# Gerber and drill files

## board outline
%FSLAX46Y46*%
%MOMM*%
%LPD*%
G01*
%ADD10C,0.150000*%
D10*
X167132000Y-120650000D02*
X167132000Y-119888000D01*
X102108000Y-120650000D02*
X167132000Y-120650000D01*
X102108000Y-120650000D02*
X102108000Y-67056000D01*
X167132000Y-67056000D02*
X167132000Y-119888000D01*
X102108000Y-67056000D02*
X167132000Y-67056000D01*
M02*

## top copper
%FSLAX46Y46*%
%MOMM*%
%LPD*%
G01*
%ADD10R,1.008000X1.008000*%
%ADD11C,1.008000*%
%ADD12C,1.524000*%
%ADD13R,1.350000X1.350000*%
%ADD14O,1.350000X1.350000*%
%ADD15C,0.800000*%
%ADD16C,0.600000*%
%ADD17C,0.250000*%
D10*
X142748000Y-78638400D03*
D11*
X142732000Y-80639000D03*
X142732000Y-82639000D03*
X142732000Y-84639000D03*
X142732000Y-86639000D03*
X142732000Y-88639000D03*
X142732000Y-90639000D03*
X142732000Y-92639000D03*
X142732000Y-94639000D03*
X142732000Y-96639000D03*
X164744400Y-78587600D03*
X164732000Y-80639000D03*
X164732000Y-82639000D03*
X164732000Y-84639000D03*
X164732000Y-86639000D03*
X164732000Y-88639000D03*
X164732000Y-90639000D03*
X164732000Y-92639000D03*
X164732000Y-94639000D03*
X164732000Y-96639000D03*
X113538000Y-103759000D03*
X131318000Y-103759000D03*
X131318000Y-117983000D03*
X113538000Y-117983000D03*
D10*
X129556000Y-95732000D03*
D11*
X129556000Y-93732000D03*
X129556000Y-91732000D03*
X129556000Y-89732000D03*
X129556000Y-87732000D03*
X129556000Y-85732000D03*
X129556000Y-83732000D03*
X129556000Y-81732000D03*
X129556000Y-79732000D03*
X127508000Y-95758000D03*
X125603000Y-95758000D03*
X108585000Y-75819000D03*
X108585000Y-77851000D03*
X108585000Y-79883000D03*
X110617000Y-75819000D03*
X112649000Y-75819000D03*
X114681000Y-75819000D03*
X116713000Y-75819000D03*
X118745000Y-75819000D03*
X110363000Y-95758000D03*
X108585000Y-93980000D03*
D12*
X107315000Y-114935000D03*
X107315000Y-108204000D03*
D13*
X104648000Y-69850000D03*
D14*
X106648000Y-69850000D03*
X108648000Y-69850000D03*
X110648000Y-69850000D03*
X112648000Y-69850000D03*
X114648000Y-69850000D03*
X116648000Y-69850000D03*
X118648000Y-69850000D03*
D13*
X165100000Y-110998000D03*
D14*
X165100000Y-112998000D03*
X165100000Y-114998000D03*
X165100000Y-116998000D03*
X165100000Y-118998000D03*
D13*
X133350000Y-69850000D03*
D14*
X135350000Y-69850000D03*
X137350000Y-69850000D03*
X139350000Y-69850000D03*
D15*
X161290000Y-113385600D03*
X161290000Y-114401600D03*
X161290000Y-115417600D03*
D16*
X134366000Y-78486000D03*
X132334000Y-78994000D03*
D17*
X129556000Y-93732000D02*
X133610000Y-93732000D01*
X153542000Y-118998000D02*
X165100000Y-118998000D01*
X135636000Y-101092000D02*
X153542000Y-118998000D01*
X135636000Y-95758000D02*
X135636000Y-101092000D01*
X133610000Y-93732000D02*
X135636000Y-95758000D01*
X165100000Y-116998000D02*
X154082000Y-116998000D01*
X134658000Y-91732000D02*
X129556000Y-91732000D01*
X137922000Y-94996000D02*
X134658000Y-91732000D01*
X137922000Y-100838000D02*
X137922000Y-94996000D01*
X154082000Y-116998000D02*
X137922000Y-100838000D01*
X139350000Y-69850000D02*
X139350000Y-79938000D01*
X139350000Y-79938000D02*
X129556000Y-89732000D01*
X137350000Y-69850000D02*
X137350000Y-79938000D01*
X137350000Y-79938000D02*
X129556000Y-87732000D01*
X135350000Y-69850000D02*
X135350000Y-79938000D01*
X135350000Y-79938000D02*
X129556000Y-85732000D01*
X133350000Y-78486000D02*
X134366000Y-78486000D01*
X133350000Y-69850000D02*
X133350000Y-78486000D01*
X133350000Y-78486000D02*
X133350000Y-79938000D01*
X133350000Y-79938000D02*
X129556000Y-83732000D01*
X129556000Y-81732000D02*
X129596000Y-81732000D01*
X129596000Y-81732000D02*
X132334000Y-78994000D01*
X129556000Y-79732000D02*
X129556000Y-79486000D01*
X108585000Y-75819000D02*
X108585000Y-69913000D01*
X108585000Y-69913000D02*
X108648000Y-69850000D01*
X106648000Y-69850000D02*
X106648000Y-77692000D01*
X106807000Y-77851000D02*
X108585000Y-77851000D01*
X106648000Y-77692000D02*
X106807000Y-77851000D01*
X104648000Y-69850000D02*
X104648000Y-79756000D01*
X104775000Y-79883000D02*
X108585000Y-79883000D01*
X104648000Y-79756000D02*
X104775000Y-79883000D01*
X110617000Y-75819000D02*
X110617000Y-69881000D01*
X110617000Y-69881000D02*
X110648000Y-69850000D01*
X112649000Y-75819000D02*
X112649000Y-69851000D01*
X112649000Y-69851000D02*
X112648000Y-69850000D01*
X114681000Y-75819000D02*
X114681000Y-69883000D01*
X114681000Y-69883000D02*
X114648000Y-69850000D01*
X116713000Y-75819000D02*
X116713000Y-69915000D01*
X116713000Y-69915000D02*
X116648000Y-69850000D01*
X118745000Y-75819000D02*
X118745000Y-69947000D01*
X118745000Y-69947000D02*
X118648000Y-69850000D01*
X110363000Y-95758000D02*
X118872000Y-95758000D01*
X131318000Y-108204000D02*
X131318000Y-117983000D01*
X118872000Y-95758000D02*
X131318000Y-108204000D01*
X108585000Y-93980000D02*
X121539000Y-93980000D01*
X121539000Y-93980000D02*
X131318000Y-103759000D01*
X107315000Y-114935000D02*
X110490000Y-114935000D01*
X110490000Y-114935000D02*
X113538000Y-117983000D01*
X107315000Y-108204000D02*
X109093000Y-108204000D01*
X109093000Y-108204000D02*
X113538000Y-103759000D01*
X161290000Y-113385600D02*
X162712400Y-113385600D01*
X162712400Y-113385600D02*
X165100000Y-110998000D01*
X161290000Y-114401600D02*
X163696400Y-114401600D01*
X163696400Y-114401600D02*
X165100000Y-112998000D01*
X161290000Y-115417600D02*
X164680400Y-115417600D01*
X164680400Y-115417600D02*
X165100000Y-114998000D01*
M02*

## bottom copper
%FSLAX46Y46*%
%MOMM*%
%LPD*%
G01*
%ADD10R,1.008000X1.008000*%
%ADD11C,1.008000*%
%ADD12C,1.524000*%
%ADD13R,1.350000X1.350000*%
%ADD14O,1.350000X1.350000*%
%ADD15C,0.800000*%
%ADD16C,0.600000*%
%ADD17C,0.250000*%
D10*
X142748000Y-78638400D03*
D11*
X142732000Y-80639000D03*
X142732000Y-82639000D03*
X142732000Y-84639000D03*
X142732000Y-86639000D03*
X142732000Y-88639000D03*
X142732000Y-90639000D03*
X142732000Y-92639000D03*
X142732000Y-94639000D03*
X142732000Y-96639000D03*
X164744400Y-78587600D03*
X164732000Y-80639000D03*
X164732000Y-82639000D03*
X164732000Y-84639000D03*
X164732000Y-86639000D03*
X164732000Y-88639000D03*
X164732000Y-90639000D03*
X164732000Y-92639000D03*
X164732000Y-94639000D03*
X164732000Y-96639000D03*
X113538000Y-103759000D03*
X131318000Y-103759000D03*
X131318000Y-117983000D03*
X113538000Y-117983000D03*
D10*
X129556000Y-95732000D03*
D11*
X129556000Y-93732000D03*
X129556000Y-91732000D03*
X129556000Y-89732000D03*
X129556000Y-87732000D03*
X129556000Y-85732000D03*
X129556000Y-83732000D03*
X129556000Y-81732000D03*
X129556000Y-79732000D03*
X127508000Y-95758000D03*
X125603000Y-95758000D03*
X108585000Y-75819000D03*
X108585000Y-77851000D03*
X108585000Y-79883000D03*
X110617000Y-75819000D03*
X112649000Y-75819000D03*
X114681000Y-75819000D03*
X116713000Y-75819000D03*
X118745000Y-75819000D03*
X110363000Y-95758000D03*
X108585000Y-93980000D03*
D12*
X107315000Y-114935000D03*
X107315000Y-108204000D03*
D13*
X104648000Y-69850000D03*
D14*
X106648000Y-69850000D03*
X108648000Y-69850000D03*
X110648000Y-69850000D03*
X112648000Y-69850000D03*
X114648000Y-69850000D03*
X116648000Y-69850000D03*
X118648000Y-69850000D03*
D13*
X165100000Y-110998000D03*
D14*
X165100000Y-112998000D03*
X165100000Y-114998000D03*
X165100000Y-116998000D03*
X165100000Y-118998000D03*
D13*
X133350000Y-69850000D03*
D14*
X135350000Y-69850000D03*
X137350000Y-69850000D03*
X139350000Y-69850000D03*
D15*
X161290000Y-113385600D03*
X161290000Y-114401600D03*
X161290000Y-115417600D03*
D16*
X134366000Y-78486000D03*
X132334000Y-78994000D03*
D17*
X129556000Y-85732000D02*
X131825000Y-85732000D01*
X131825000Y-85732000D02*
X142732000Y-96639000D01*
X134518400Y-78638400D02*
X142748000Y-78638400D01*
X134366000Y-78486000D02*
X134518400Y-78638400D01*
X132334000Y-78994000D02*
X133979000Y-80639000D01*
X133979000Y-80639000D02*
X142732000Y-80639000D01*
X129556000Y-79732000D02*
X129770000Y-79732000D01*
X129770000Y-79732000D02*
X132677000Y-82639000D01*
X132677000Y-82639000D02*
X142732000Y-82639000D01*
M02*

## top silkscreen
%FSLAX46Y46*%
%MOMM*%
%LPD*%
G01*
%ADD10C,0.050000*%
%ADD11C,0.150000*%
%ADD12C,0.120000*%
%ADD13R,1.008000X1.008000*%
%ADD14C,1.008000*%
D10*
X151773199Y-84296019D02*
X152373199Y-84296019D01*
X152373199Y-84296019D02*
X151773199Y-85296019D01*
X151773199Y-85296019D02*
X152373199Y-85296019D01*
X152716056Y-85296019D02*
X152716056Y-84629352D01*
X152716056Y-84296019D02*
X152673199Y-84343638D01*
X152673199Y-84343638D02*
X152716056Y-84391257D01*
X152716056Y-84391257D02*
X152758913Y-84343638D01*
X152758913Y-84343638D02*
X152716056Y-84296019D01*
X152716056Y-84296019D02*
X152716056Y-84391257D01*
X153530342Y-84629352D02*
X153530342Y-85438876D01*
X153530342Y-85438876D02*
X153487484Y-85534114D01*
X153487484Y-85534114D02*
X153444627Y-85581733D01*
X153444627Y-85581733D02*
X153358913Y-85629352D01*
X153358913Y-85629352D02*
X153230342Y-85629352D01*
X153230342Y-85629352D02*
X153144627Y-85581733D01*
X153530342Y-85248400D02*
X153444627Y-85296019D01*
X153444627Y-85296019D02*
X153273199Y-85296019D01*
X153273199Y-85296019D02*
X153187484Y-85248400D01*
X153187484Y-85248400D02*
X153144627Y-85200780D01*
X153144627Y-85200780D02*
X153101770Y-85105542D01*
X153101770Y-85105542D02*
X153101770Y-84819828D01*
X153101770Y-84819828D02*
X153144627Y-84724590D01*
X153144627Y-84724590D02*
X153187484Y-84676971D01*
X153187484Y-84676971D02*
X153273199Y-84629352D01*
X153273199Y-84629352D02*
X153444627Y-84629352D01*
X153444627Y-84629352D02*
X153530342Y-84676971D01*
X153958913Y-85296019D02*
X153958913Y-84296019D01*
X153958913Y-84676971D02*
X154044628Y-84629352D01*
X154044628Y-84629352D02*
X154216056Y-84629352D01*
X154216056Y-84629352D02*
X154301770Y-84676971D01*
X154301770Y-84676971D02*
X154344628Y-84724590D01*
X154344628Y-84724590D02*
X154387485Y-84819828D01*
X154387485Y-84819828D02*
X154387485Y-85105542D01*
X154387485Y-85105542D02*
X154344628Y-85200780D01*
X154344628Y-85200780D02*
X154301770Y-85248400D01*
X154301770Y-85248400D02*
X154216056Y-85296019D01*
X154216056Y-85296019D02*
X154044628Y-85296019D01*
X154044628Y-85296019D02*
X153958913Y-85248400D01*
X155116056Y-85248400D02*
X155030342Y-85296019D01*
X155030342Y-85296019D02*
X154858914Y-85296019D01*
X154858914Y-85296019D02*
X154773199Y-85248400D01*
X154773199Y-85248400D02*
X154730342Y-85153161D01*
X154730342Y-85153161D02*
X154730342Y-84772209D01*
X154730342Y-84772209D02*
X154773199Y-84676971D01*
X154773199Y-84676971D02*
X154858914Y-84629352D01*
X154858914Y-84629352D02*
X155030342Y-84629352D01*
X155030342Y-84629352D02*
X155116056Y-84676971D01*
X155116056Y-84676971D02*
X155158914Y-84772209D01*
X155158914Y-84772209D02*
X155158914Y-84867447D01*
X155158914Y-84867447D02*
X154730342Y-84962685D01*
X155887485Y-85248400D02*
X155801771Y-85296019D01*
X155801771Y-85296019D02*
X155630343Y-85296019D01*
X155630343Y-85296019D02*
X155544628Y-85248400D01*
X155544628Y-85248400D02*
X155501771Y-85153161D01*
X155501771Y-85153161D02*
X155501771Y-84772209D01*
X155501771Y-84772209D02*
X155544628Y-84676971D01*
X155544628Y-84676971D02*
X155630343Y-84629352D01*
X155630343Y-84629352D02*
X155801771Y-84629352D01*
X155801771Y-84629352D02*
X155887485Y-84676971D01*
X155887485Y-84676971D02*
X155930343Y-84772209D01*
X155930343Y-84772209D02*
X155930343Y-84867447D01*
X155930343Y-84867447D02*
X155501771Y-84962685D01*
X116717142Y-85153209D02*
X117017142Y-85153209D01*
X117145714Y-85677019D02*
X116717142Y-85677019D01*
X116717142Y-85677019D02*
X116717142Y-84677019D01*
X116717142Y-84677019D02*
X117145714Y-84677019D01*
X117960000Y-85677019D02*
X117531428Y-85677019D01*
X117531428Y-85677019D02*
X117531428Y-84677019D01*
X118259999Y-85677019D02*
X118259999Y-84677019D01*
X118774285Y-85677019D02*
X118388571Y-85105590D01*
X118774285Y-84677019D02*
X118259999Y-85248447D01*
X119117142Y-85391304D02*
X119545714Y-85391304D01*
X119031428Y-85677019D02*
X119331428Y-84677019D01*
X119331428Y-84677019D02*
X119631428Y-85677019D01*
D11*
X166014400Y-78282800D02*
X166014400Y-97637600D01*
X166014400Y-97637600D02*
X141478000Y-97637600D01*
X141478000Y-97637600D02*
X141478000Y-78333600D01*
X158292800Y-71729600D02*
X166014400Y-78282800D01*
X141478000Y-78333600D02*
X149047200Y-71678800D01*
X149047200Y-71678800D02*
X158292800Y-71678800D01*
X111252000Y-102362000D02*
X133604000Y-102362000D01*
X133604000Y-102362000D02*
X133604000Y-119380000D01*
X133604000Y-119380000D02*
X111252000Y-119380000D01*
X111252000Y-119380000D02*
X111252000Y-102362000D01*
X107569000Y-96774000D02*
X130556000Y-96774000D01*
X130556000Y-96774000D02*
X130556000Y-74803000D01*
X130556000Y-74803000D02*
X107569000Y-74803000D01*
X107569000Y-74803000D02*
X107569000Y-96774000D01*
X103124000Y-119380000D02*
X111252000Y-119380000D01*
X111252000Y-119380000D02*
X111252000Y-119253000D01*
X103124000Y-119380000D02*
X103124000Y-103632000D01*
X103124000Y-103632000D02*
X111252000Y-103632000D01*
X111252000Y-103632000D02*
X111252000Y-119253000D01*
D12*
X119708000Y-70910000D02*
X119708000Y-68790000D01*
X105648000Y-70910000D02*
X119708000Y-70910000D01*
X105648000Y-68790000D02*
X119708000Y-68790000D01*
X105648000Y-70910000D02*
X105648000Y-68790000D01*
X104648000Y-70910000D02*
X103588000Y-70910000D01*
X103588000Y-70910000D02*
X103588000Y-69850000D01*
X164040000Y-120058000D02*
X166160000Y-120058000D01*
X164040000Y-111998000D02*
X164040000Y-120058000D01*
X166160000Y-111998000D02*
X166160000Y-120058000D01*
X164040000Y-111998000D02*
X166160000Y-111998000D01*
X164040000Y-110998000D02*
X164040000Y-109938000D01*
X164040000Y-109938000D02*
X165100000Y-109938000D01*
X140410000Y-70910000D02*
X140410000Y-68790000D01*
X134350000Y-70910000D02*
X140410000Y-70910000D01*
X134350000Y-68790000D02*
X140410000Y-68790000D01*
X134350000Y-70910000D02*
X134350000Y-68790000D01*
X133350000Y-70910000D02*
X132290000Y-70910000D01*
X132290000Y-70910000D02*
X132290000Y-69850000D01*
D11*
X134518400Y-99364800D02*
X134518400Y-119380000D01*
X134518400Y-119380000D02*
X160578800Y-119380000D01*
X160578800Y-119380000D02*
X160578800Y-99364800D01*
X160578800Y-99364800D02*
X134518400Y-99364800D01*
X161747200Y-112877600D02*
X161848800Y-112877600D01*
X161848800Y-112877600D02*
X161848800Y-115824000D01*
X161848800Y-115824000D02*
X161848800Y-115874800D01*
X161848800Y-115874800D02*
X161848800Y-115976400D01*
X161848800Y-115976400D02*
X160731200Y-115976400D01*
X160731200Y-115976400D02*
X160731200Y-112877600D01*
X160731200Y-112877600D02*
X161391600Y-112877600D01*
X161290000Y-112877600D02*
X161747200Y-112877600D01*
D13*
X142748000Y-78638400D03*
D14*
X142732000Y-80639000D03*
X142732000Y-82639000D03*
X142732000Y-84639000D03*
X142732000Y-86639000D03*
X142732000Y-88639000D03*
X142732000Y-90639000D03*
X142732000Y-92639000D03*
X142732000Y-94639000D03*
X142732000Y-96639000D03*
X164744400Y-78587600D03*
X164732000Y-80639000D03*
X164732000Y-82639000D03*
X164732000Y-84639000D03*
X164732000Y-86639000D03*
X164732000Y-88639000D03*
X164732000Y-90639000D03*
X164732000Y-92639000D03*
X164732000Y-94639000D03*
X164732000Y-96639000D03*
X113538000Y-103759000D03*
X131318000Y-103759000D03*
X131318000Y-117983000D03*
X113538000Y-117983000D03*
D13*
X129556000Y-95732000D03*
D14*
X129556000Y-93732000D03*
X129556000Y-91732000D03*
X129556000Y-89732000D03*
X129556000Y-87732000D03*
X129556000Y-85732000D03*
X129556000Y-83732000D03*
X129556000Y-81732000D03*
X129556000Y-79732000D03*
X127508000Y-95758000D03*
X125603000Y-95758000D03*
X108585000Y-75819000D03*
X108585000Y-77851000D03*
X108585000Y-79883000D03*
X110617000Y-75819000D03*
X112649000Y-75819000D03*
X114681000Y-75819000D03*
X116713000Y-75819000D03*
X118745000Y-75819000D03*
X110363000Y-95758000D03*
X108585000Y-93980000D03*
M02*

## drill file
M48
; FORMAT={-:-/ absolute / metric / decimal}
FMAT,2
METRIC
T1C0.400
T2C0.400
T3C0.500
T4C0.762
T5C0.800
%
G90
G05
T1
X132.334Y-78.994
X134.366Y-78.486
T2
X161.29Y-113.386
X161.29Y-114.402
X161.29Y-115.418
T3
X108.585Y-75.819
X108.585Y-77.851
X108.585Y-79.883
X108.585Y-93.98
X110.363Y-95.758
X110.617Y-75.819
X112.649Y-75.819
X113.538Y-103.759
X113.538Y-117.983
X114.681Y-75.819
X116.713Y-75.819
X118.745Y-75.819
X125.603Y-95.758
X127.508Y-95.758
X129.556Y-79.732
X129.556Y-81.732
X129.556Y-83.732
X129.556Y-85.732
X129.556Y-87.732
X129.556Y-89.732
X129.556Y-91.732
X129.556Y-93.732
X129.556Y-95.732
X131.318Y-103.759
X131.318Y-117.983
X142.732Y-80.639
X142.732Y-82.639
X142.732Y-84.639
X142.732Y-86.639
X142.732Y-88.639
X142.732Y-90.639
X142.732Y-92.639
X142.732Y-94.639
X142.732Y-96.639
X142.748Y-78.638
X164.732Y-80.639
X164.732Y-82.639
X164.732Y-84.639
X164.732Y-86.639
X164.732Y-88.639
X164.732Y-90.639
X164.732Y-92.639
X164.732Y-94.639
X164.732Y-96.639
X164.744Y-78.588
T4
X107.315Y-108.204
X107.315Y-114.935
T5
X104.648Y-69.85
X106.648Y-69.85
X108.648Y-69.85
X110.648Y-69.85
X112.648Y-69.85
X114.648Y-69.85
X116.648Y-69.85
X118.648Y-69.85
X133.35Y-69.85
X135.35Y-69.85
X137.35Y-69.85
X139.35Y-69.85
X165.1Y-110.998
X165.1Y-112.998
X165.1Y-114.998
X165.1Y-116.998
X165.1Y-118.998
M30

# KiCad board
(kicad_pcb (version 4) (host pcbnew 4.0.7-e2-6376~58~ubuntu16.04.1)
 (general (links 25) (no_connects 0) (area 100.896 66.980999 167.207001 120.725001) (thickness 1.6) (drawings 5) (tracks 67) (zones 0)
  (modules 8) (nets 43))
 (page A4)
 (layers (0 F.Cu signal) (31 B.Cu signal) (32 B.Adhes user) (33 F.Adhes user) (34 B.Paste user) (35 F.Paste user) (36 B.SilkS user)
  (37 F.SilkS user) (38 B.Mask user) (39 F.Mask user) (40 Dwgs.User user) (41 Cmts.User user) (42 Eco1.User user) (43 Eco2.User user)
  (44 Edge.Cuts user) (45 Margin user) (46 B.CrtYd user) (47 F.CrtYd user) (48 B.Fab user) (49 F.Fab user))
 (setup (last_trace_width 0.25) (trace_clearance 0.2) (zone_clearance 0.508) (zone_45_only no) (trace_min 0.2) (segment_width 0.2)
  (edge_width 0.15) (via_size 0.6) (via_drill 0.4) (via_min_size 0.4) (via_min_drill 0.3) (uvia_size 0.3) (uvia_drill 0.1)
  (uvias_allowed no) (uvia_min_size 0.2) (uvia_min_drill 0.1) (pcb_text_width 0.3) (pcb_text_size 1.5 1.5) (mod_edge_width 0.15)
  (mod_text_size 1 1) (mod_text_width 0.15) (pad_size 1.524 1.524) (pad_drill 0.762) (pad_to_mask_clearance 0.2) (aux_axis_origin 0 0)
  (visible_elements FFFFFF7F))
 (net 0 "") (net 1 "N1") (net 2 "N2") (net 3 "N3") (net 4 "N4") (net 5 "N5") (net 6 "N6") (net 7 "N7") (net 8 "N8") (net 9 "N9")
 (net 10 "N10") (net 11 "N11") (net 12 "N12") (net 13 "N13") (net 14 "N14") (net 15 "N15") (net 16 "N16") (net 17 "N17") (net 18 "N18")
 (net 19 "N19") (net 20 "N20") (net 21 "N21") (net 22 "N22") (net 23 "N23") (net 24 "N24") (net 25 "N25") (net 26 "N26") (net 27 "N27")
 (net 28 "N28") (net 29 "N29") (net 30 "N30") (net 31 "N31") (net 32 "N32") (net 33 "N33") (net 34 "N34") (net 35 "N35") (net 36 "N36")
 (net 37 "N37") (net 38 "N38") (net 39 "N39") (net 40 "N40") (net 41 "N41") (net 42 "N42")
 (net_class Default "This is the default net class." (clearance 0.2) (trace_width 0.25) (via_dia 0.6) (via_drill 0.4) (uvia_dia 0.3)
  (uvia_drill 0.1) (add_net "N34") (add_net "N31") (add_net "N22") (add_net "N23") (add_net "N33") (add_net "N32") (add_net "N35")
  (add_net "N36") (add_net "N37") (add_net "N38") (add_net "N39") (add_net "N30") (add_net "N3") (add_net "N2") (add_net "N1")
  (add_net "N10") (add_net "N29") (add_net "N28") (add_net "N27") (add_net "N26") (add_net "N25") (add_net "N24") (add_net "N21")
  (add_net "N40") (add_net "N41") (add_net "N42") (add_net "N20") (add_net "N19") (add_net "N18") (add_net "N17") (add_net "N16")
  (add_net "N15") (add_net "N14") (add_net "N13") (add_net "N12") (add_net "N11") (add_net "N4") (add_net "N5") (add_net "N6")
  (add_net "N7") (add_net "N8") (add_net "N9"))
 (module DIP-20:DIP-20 (layer F.Cu) (at 141.478 104.648)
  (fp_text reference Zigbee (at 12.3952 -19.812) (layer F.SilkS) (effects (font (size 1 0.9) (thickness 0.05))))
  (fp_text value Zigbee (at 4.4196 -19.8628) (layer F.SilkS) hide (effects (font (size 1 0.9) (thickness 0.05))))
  (fp_line (start 24.5364 -26.3652) (end 24.5364 -7.0104) (layer F.SilkS) (width 0.15))
  (fp_line (start 24.5364 -7.0104) (end 0 -7.0104) (layer F.SilkS) (width 0.15))
  (fp_line (start 0 -7.0104) (end 0 -26.3144) (layer F.SilkS) (width 0.15))
  (fp_line (start 16.8148 -32.9184) (end 24.5364 -26.3652) (layer F.SilkS) (width 0.15))
  (fp_line (start 0 -26.3144) (end 7.5692 -32.9692) (layer F.SilkS) (width 0.15))
  (fp_line (start 7.5692 -32.9692) (end 16.8148 -32.9692) (layer F.SilkS) (width 0.15))
  (pad 1 thru_hole rect (at 1.27 -26.0096) (size 1.008 1.008) (drill 0.5) (layers *.Cu *.Mask F.SilkS) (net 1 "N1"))
  (pad 2 thru_hole circle (at 1.254 -24.009) (size 1.008 1.008) (drill 0.5) (layers *.Cu *.Mask F.SilkS) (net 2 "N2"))
  (pad 3 thru_hole circle (at 1.254 -22.009) (size 1.008 1.008) (drill 0.5) (layers *.Cu *.Mask F.SilkS) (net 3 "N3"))
  (pad 4 thru_hole circle (at 1.254 -20.009) (size 1.008 1.008) (drill 0.5) (layers *.Cu *.Mask F.SilkS) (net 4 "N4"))
  (pad 5 thru_hole circle (at 1.254 -18.009) (size 1.008 1.008) (drill 0.5) (layers *.Cu *.Mask F.SilkS) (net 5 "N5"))
  (pad 6 thru_hole circle (at 1.254 -16.009) (size 1.008 1.008) (drill 0.5) (layers *.Cu *.Mask F.SilkS) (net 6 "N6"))
  (pad 7 thru_hole circle (at 1.254 -14.009) (size 1.008 1.008) (drill 0.5) (layers *.Cu *.Mask F.SilkS) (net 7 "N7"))
  (pad 8 thru_hole circle (at 1.254 -12.009) (size 1.008 1.008) (drill 0.5) (layers *.Cu *.Mask F.SilkS) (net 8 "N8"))
  (pad 9 thru_hole circle (at 1.254 -10.009) (size 1.008 1.008) (drill 0.5) (layers *.Cu *.Mask F.SilkS) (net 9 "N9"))
  (pad 10 thru_hole circle (at 1.254 -8.009) (size 1.008 1.008) (drill 0.5) (layers *.Cu *.Mask F.SilkS) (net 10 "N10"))
  (pad 20 thru_hole circle (at 23.2664 -26.0604) (size 1.008 1.008) (drill 0.5) (layers *.Cu *.Mask F.SilkS) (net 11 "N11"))
  (pad 19 thru_hole circle (at 23.254 -24.009) (size 1.008 1.008) (drill 0.5) (layers *.Cu *.Mask F.SilkS) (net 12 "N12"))
  (pad 18 thru_hole circle (at 23.254 -22.009) (size 1.008 1.008) (drill 0.5) (layers *.Cu *.Mask F.SilkS) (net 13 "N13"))
  (pad 17 thru_hole circle (at 23.254 -20.009) (size 1.008 1.008) (drill 0.5) (layers *.Cu *.Mask F.SilkS) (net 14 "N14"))
  (pad 16 thru_hole circle (at 23.254 -18.009) (size 1.008 1.008) (drill 0.5) (layers *.Cu *.Mask F.SilkS) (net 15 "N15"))
  (pad 15 thru_hole circle (at 23.254 -16.009) (size 1.008 1.008) (drill 0.5) (layers *.Cu *.Mask F.SilkS) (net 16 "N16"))
  (pad 14 thru_hole circle (at 23.254 -14.009) (size 1.008 1.008) (drill 0.5) (layers *.Cu *.Mask F.SilkS) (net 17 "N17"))
  (pad 13 thru_hole circle (at 23.254 -12.009) (size 1.008 1.008) (drill 0.5) (layers *.Cu *.Mask F.SilkS) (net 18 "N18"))
  (pad 12 thru_hole circle (at 23.254 -10.009) (size 1.008 1.008) (drill 0.5) (layers *.Cu *.Mask F.SilkS) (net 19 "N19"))
  (pad 11 thru_hole circle (at 23.254 -8.009) (size 1.008 1.008) (drill 0.5) (layers *.Cu *.Mask F.SilkS) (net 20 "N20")))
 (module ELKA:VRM (layer F.Cu) (at 118.872 100.838)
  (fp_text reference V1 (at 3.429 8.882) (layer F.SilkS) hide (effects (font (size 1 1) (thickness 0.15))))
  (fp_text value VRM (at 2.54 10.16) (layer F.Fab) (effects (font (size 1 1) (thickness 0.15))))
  (fp_line (start -7.62 1.524) (end 14.732 1.524) (layer F.SilkS) (width 0.15))
  (fp_line (start 14.732 1.524) (end 14.732 18.542) (layer F.SilkS) (width 0.15))
  (fp_line (start 14.732 18.542) (end -7.62 18.542) (layer F.SilkS) (width 0.15))
  (fp_line (start -7.62 18.542) (end -7.62 1.524) (layer F.SilkS) (width 0.15))
  (pad 2 thru_hole circle (at -5.334 2.921) (size 1.008 1.008) (drill 0.5) (layers *.Cu *.Mask F.SilkS) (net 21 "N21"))
  (pad 4 thru_hole circle (at 12.446 2.921) (size 1.008 1.008) (drill 0.5) (layers *.Cu *.Mask F.SilkS) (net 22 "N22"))
  (pad 3 thru_hole circle (at 12.446 17.145) (size 1.008 1.008) (drill 0.5) (layers *.Cu *.Mask F.SilkS) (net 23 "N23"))
  (pad 1 thru_hole circle (at -5.334 17.145) (size 1.008 1.008) (drill 0.5) (layers *.Cu *.Mask F.SilkS) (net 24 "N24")))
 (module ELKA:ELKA (layer F.Cu) (at 118.11 72.39 180)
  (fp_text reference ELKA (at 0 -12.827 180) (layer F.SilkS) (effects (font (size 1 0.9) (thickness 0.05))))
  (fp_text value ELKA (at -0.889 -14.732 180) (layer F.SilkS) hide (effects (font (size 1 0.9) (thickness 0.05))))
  (fp_line (start 10.541 -24.384) (end -12.446 -24.384) (layer F.SilkS) (width 0.15))
  (fp_line (start -12.446 -24.384) (end -12.446 -2.413) (layer F.SilkS) (width 0.15))
  (fp_line (start -12.446 -2.413) (end 10.541 -2.413) (layer F.SilkS) (width 0.15))
  (fp_line (start 10.541 -2.413) (end 10.541 -24.384) (layer F.SilkS) (width 0.15))
  (pad I thru_hole rect (at -11.446 -23.342 180) (size 1.008 1.008) (drill 0.5) (layers *.Cu *.Mask F.SilkS) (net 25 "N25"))
  (pad H thru_hole circle (at -11.446 -21.342 180) (size 1.008 1.008) (drill 0.5) (layers *.Cu *.Mask F.SilkS) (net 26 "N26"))
  (pad G thru_hole circle (at -11.446 -19.342 180) (size 1.008 1.008) (drill 0.5) (layers *.Cu *.Mask F.SilkS) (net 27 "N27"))
  (pad F thru_hole circle (at -11.446 -17.342 180) (size 1.008 1.008) (drill 0.5) (layers *.Cu *.Mask F.SilkS) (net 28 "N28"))
  (pad E thru_hole circle (at -11.446 -15.342 180) (size 1.008 1.008) (drill 0.5) (layers *.Cu *.Mask F.SilkS) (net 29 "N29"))
  (pad D thru_hole circle (at -11.446 -13.342 180) (size 1.008 1.008) (drill 0.5) (layers *.Cu *.Mask F.SilkS) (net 10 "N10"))
  (pad C thru_hole circle (at -11.446 -11.342 180) (size 1.008 1.008) (drill 0.5) (layers *.Cu *.Mask F.SilkS) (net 1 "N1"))
  (pad B thru_hole circle (at -11.446 -9.342 180) (size 1.008 1.008) (drill 0.5) (layers *.Cu *.Mask F.SilkS) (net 2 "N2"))
  (pad A thru_hole circle (at -11.446 -7.342 180) (size 1.008 1.008) (drill 0.5) (layers *.Cu *.Mask F.SilkS) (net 3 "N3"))
  (pad 9 thru_hole circle (at -9.398 -23.368 180) (size 1.008 1.008) (drill 0.5) (layers *.Cu *.Mask F.SilkS) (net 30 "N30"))
  (pad 10 thru_hole circle (at -7.493 -23.368 180) (size 1.008 1.008) (drill 0.5) (layers *.Cu *.Mask F.SilkS) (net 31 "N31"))
  (pad 3 thru_hole circle (at 9.525 -3.429 180) (size 1.008 1.008) (drill 0.5) (layers *.Cu *.Mask F.SilkS) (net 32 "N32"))
  (pad 2 thru_hole circle (at 9.525 -5.461 180) (size 1.008 1.008) (drill 0.5) (layers *.Cu *.Mask F.SilkS) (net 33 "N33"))
  (pad 1 thru_hole circle (at 9.525 -7.493 180) (size 1.008 1.008) (drill 0.5) (layers *.Cu *.Mask F.SilkS) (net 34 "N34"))
  (pad 4 thru_hole circle (at 7.493 -3.429 180) (size 1.008 1.008) (drill 0.5) (layers *.Cu *.Mask F.SilkS) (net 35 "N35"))
  (pad 5 thru_hole circle (at 5.461 -3.429 180) (size 1.008 1.008) (drill 0.5) (layers *.Cu *.Mask F.SilkS) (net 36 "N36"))
  (pad 6 thru_hole circle (at 3.429 -3.429 180) (size 1.008 1.008) (drill 0.5) (layers *.Cu *.Mask F.SilkS) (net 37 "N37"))
  (pad 7 thru_hole circle (at 1.397 -3.429 180) (size 1.008 1.008) (drill 0.5) (layers *.Cu *.Mask F.SilkS) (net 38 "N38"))
  (pad 8 thru_hole circle (at -0.635 -3.429 180) (size 1.008 1.008) (drill 0.5) (layers *.Cu *.Mask F.SilkS) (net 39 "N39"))
  (pad 12 thru_hole circle (at 7.747 -23.368 180) (size 1.008 1.008) (drill 0.5) (layers *.Cu *.Mask F.SilkS) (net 23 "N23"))
  (pad 11 thru_hole circle (at 9.525 -21.59 180) (size 1.008 1.008) (drill 0.5) (layers *.Cu *.Mask F.SilkS) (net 22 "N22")))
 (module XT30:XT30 (layer F.Cu) (at 101.346 113.538 90)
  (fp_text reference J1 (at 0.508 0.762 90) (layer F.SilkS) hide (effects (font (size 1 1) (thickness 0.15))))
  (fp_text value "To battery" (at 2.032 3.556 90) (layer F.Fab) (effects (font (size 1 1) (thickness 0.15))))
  (fp_line (start -5.842 1.778) (end -5.842 9.906) (layer F.SilkS) (width 0.15))
  (fp_line (start -5.842 9.906) (end -5.715 9.906) (layer F.SilkS) (width 0.15))
  (fp_line (start -5.842 1.778) (end 9.906 1.778) (layer F.SilkS) (width 0.15))
  (fp_line (start 9.906 1.778) (end 9.906 9.906) (layer F.SilkS) (width 0.15))
  (fp_line (start 9.906 9.906) (end -5.715 9.906) (layer F.SilkS) (width 0.15))
  (pad 1 thru_hole circle (at -1.397 5.969 90) (size 1.524 1.524) (drill 0.762) (layers *.Cu *.Mask) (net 24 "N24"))
  (pad 2 thru_hole circle (at 5.334 5.969 90) (size 1.524 1.524) (drill 0.762) (layers *.Cu *.Mask) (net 21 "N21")))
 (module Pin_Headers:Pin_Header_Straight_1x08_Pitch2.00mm (layer F.Cu) (at 104.648 69.85 90)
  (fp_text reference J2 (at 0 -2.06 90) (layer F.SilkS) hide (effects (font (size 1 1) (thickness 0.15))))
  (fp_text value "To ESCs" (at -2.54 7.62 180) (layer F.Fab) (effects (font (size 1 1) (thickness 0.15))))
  (fp_line (start -1.06 15.06) (end 1.06 15.06) (layer F.SilkS) (width 0.12))
  (fp_line (start -1.06 1) (end -1.06 15.06) (layer F.SilkS) (width 0.12))
  (fp_line (start 1.06 1) (end 1.06 15.06) (layer F.SilkS) (width 0.12))
  (fp_line (start -1.06 1) (end 1.06 1) (layer F.SilkS) (width 0.12))
  (fp_line (start -1.06 0) (end -1.06 -1.06) (layer F.SilkS) (width 0.12))
  (fp_line (start -1.06 -1.06) (end 0 -1.06) (layer F.SilkS) (width 0.12))
  (pad 1 thru_hole rect (at 0 0 90) (size 1.35 1.35) (drill 0.8) (layers *.Cu *.Mask) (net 34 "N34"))
  (pad 2 thru_hole oval (at 0 2 90) (size 1.35 1.35) (drill 0.8) (layers *.Cu *.Mask) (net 33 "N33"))
  (pad 3 thru_hole oval (at 0 4 90) (size 1.35 1.35) (drill 0.8) (layers *.Cu *.Mask) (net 32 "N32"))
  (pad 4 thru_hole oval (at 0 6 90) (size 1.35 1.35) (drill 0.8) (layers *.Cu *.Mask) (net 35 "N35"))
  (pad 5 thru_hole oval (at 0 8 90) (size 1.35 1.35) (drill 0.8) (layers *.Cu *.Mask) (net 36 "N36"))
  (pad 6 thru_hole oval (at 0 10 90) (size 1.35 1.35) (drill 0.8) (layers *.Cu *.Mask) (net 37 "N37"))
  (pad 7 thru_hole oval (at 0 12 90) (size 1.35 1.35) (drill 0.8) (layers *.Cu *.Mask) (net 38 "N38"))
  (pad 8 thru_hole oval (at 0 14 90) (size 1.35 1.35) (drill 0.8) (layers *.Cu *.Mask) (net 39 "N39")))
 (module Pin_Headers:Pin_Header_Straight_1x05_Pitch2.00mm (layer F.Cu) (at 165.1 110.998)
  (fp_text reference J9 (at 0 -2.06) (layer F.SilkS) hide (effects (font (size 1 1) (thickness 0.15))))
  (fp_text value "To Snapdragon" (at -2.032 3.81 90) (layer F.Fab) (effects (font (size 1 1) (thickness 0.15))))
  (fp_line (start -1.06 9.06) (end 1.06 9.06) (layer F.SilkS) (width 0.12))
  (fp_line (start -1.06 1) (end -1.06 9.06) (layer F.SilkS) (width 0.12))
  (fp_line (start 1.06 1) (end 1.06 9.06) (layer F.SilkS) (width 0.12))
  (fp_line (start -1.06 1) (end 1.06 1) (layer F.SilkS) (width 0.12))
  (fp_line (start -1.06 0) (end -1.06 -1.06) (layer F.SilkS) (width 0.12))
  (fp_line (start -1.06 -1.06) (end 0 -1.06) (layer F.SilkS) (width 0.12))
  (pad 1 thru_hole rect (at 0 0) (size 1.35 1.35) (drill 0.8) (layers *.Cu *.Mask) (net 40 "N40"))
  (pad 2 thru_hole oval (at 0 2) (size 1.35 1.35) (drill 0.8) (layers *.Cu *.Mask) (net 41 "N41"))
  (pad 3 thru_hole oval (at 0 4) (size 1.35 1.35) (drill 0.8) (layers *.Cu *.Mask) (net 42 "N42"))
  (pad 4 thru_hole oval (at 0 6) (size 1.35 1.35) (drill 0.8) (layers *.Cu *.Mask) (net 27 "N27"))
  (pad 5 thru_hole oval (at 0 8) (size 1.35 1.35) (drill 0.8) (layers *.Cu *.Mask) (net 26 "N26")))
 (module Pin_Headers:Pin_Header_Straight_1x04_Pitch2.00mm (layer F.Cu) (at 133.35 69.85 90)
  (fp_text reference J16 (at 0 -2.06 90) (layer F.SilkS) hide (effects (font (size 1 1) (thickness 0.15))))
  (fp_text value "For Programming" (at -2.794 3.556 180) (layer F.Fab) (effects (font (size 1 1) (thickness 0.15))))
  (fp_line (start -1.06 7.06) (end 1.06 7.06) (layer F.SilkS) (width 0.12))
  (fp_line (start -1.06 1) (end -1.06 7.06) (layer F.SilkS) (width 0.12))
  (fp_line (start 1.06 1) (end 1.06 7.06) (layer F.SilkS) (width 0.12))
  (fp_line (start -1.06 1) (end 1.06 1) (layer F.SilkS) (width 0.12))
  (fp_line (start -1.06 0) (end -1.06 -1.06) (layer F.SilkS) (width 0.12))
  (fp_line (start -1.06 -1.06) (end 0 -1.06) (layer F.SilkS) (width 0.12))
  (pad 1 thru_hole rect (at 0 0 90) (size 1.35 1.35) (drill 0.8) (layers *.Cu *.Mask) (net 1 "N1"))
  (pad 2 thru_hole oval (at 0 2 90) (size 1.35 1.35) (drill 0.8) (layers *.Cu *.Mask) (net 10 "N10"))
  (pad 3 thru_hole oval (at 0 4 90) (size 1.35 1.35) (drill 0.8) (layers *.Cu *.Mask) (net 29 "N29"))
  (pad 4 thru_hole oval (at 0 6 90) (size 1.35 1.35) (drill 0.8) (layers *.Cu *.Mask) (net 28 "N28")))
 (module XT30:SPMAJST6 (layer F.Cu) (at 164.084 115.316 270)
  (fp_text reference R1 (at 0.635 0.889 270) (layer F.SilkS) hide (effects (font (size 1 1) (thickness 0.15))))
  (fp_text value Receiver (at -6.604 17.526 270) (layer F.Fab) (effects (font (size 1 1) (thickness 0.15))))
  (fp_line (start -15.9512 29.5656) (end 4.064 29.5656) (layer F.SilkS) (width 0.15))
  (fp_line (start 4.064 29.5656) (end 4.064 3.5052) (layer F.SilkS) (width 0.15))
  (fp_line (start 4.064 3.5052) (end -15.9512 3.5052) (layer F.SilkS) (width 0.15))
  (fp_line (start -15.9512 3.5052) (end -15.9512 29.5656) (layer F.SilkS) (width 0.15))
  (fp_line (start -2.4384 2.3368) (end -2.4384 2.2352) (layer F.SilkS) (width 0.15))
  (fp_line (start -2.4384 2.2352) (end 0.508 2.2352) (layer F.SilkS) (width 0.15))
  (fp_line (start 0.508 2.2352) (end 0.5588 2.2352) (layer F.SilkS) (width 0.15))
  (fp_line (start 0.5588 2.2352) (end 0.6604 2.2352) (layer F.SilkS) (width 0.15))
  (fp_line (start 0.6604 2.2352) (end 0.6604 3.3528) (layer F.SilkS) (width 0.15))
  (fp_line (start 0.6604 3.3528) (end -2.4384 3.3528) (layer F.SilkS) (width 0.15))
  (fp_line (start -2.4384 3.3528) (end -2.4384 2.6924) (layer F.SilkS) (width 0.15))
  (fp_line (start -2.4384 2.794) (end -2.4384 2.3368) (layer F.SilkS) (width 0.15))
  (pad 1 thru_hole circle (at -1.9304 2.794 270) (size 0.8 0.8) (drill 0.4) (layers *.Cu *.Mask) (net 40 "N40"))
  (pad 2 thru_hole circle (at -0.9144 2.794 270) (size 0.8 0.8) (drill 0.4) (layers *.Cu *.Mask) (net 41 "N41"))
  (pad 3 thru_hole circle (at 0.1016 2.794 270) (size 0.8 0.8) (drill 0.4) (layers *.Cu *.Mask) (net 42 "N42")))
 (gr_line (start 167.132 120.65) (end 167.132 119.888) (angle 90) (layer Edge.Cuts) (width 0.15))
 (gr_line (start 102.108 120.65) (end 167.132 120.65) (angle 90) (layer Edge.Cuts) (width 0.15))
 (gr_line (start 102.108 120.65) (end 102.108 67.056) (angle 90) (layer Edge.Cuts) (width 0.15))
 (gr_line (start 167.132 67.056) (end 167.132 119.888) (angle 90) (layer Edge.Cuts) (width 0.15))
 (gr_line (start 102.108 67.056) (end 167.132 67.056) (angle 90) (layer Edge.Cuts) (width 0.15))
 (segment (start 129.556 93.732) (end 133.61 93.732) (width 0.25) (layer F.Cu) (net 26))
 (segment (start 153.542 118.998) (end 165.1 118.998) (width 0.25) (layer F.Cu) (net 26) (status 20))
 (segment (start 135.636 101.092) (end 153.542 118.998) (width 0.25) (layer F.Cu) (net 26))
 (segment (start 135.636 95.758) (end 135.636 101.092) (width 0.25) (layer F.Cu) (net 26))
 (segment (start 133.61 93.732) (end 135.636 95.758) (width 0.25) (layer F.Cu) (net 26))
 (segment (start 165.1 116.998) (end 154.082 116.998) (width 0.25) (layer F.Cu) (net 27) (status 10))
 (segment (start 134.658 91.732) (end 129.556 91.732) (width 0.25) (layer F.Cu) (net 27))
 (segment (start 137.922 94.996) (end 134.658 91.732) (width 0.25) (layer F.Cu) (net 27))
 (segment (start 137.922 100.838) (end 137.922 94.996) (width 0.25) (layer F.Cu) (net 27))
 (segment (start 154.082 116.998) (end 137.922 100.838) (width 0.25) (layer F.Cu) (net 27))
 (segment (start 139.35 69.85) (end 139.35 79.938) (width 0.25) (layer F.Cu) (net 28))
 (segment (start 139.35 79.938) (end 129.556 89.732) (width 0.25) (layer F.Cu) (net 28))
 (segment (start 137.35 69.85) (end 137.35 79.938) (width 0.25) (layer F.Cu) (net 29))
 (segment (start 137.35 79.938) (end 129.556 87.732) (width 0.25) (layer F.Cu) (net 29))
 (segment (start 129.556 85.732) (end 131.825 85.732) (width 0.25) (layer B.Cu) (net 10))
 (segment (start 131.825 85.732) (end 142.732 96.639) (width 0.25) (layer B.Cu) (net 10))
 (segment (start 135.35 69.85) (end 135.35 79.938) (width 0.25) (layer F.Cu) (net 10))
 (segment (start 135.35 79.938) (end 129.556 85.732) (width 0.25) (layer F.Cu) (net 10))
 (segment (start 133.35 78.486) (end 134.366 78.486) (width 0.25) (layer F.Cu) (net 1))
 (segment (start 134.5184 78.6384) (end 142.748 78.6384) (width 0.25) (layer B.Cu) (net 1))
 (segment (start 134.366 78.486) (end 134.5184 78.6384) (width 0.25) (layer B.Cu) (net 1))
 (via (at 134.366 78.486) (size 0.6) (drill 0.4) (layers F.Cu B.Cu) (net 1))
 (segment (start 133.35 69.85) (end 133.35 78.486) (width 0.25) (layer F.Cu) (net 1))
 (segment (start 133.35 78.486) (end 133.35 79.938) (width 0.25) (layer F.Cu) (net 1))
 (segment (start 133.35 79.938) (end 129.556 83.732) (width 0.25) (layer F.Cu) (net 1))
 (segment (start 129.556 81.732) (end 129.596 81.732) (width 0.25) (layer F.Cu) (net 2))
 (segment (start 129.596 81.732) (end 132.334 78.994) (width 0.25) (layer F.Cu) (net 2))
 (via (at 132.334 78.994) (size 0.6) (drill 0.4) (layers F.Cu B.Cu) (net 2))
 (segment (start 132.334 78.994) (end 133.979 80.639) (width 0.25) (layer B.Cu) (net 2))
 (segment (start 133.979 80.639) (end 142.732 80.639) (width 0.25) (layer B.Cu) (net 2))
 (segment (start 129.556 79.732) (end 129.77 79.732) (width 0.25) (layer B.Cu) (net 3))
 (segment (start 129.77 79.732) (end 132.677 82.639) (width 0.25) (layer B.Cu) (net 3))
 (segment (start 132.677 82.639) (end 142.732 82.639) (width 0.25) (layer B.Cu) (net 3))
 (segment (start 129.556 79.732) (end 129.556 79.486) (width 0.25) (layer F.Cu) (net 3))
 (segment (start 108.585 75.819) (end 108.585 69.913) (width 0.25) (layer F.Cu) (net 32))
 (segment (start 108.585 69.913) (end 108.648 69.85) (width 0.25) (layer F.Cu) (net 32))
 (segment (start 106.648 69.85) (end 106.648 77.692) (width 0.25) (layer F.Cu) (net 33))
 (segment (start 106.807 77.851) (end 108.585 77.851) (width 0.25) (layer F.Cu) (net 33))
 (segment (start 106.648 77.692) (end 106.807 77.851) (width 0.25) (layer F.Cu) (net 33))
 (segment (start 104.648 69.85) (end 104.648 79.756) (width 0.25) (layer F.Cu) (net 34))
 (segment (start 104.775 79.883) (end 108.585 79.883) (width 0.25) (layer F.Cu) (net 34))
 (segment (start 104.648 79.756) (end 104.775 79.883) (width 0.25) (layer F.Cu) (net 34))
 (segment (start 110.617 75.819) (end 110.617 69.881) (width 0.25) (layer F.Cu) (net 35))
 (segment (start 110.617 69.881) (end 110.648 69.85) (width 0.25) (layer F.Cu) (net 35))
 (segment (start 112.649 75.819) (end 112.649 69.851) (width 0.25) (layer F.Cu) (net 36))
 (segment (start 112.649 69.851) (end 112.648 69.85) (width 0.25) (layer F.Cu) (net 36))
 (segment (start 114.681 75.819) (end 114.681 69.883) (width 0.25) (layer F.Cu) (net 37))
 (segment (start 114.681 69.883) (end 114.648 69.85) (width 0.25) (layer F.Cu) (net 37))
 (segment (start 116.713 75.819) (end 116.713 69.915) (width 0.25) (layer F.Cu) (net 38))
 (segment (start 116.713 69.915) (end 116.648 69.85) (width 0.25) (layer F.Cu) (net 38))
 (segment (start 118.745 75.819) (end 118.745 69.947) (width 0.25) (layer F.Cu) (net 39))
 (segment (start 118.745 69.947) (end 118.648 69.85) (width 0.25) (layer F.Cu) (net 39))
 (segment (start 110.363 95.758) (end 118.872 95.758) (width 0.25) (layer F.Cu) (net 23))
 (segment (start 131.318 108.204) (end 131.318 117.983) (width 0.25) (layer F.Cu) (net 23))
 (segment (start 118.872 95.758) (end 131.318 108.204) (width 0.25) (layer F.Cu) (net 23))
 (segment (start 108.585 93.98) (end 121.539 93.98) (width 0.25) (layer F.Cu) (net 22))
 (segment (start 121.539 93.98) (end 131.318 103.759) (width 0.25) (layer F.Cu) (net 22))
 (segment (start 107.315 114.935) (end 110.49 114.935) (width 0.25) (layer F.Cu) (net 24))
 (segment (start 110.49 114.935) (end 113.538 117.983) (width 0.25) (layer F.Cu) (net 24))
 (segment (start 107.315 108.204) (end 109.093 108.204) (width 0.25) (layer F.Cu) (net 21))
 (segment (start 109.093 108.204) (end 113.538 103.759) (width 0.25) (layer F.Cu) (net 21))
 (segment (start 161.29 113.3856) (end 162.7124 113.3856) (width 0.25) (layer F.Cu) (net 40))
 (segment (start 162.7124 113.3856) (end 165.1 110.998) (width 0.25) (layer F.Cu) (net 40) (status 20))
 (segment (start 161.29 114.4016) (end 163.6964 114.4016) (width 0.25) (layer F.Cu) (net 41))
 (segment (start 163.6964 114.4016) (end 165.1 112.998) (width 0.25) (layer F.Cu) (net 41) (status 20))
 (segment (start 161.29 115.4176) (end 164.6804 115.4176) (width 0.25) (layer F.Cu) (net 42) (status 20))
 (segment (start 164.6804 115.4176) (end 165.1 114.998) (width 0.25) (layer F.Cu) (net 42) (status 30)))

